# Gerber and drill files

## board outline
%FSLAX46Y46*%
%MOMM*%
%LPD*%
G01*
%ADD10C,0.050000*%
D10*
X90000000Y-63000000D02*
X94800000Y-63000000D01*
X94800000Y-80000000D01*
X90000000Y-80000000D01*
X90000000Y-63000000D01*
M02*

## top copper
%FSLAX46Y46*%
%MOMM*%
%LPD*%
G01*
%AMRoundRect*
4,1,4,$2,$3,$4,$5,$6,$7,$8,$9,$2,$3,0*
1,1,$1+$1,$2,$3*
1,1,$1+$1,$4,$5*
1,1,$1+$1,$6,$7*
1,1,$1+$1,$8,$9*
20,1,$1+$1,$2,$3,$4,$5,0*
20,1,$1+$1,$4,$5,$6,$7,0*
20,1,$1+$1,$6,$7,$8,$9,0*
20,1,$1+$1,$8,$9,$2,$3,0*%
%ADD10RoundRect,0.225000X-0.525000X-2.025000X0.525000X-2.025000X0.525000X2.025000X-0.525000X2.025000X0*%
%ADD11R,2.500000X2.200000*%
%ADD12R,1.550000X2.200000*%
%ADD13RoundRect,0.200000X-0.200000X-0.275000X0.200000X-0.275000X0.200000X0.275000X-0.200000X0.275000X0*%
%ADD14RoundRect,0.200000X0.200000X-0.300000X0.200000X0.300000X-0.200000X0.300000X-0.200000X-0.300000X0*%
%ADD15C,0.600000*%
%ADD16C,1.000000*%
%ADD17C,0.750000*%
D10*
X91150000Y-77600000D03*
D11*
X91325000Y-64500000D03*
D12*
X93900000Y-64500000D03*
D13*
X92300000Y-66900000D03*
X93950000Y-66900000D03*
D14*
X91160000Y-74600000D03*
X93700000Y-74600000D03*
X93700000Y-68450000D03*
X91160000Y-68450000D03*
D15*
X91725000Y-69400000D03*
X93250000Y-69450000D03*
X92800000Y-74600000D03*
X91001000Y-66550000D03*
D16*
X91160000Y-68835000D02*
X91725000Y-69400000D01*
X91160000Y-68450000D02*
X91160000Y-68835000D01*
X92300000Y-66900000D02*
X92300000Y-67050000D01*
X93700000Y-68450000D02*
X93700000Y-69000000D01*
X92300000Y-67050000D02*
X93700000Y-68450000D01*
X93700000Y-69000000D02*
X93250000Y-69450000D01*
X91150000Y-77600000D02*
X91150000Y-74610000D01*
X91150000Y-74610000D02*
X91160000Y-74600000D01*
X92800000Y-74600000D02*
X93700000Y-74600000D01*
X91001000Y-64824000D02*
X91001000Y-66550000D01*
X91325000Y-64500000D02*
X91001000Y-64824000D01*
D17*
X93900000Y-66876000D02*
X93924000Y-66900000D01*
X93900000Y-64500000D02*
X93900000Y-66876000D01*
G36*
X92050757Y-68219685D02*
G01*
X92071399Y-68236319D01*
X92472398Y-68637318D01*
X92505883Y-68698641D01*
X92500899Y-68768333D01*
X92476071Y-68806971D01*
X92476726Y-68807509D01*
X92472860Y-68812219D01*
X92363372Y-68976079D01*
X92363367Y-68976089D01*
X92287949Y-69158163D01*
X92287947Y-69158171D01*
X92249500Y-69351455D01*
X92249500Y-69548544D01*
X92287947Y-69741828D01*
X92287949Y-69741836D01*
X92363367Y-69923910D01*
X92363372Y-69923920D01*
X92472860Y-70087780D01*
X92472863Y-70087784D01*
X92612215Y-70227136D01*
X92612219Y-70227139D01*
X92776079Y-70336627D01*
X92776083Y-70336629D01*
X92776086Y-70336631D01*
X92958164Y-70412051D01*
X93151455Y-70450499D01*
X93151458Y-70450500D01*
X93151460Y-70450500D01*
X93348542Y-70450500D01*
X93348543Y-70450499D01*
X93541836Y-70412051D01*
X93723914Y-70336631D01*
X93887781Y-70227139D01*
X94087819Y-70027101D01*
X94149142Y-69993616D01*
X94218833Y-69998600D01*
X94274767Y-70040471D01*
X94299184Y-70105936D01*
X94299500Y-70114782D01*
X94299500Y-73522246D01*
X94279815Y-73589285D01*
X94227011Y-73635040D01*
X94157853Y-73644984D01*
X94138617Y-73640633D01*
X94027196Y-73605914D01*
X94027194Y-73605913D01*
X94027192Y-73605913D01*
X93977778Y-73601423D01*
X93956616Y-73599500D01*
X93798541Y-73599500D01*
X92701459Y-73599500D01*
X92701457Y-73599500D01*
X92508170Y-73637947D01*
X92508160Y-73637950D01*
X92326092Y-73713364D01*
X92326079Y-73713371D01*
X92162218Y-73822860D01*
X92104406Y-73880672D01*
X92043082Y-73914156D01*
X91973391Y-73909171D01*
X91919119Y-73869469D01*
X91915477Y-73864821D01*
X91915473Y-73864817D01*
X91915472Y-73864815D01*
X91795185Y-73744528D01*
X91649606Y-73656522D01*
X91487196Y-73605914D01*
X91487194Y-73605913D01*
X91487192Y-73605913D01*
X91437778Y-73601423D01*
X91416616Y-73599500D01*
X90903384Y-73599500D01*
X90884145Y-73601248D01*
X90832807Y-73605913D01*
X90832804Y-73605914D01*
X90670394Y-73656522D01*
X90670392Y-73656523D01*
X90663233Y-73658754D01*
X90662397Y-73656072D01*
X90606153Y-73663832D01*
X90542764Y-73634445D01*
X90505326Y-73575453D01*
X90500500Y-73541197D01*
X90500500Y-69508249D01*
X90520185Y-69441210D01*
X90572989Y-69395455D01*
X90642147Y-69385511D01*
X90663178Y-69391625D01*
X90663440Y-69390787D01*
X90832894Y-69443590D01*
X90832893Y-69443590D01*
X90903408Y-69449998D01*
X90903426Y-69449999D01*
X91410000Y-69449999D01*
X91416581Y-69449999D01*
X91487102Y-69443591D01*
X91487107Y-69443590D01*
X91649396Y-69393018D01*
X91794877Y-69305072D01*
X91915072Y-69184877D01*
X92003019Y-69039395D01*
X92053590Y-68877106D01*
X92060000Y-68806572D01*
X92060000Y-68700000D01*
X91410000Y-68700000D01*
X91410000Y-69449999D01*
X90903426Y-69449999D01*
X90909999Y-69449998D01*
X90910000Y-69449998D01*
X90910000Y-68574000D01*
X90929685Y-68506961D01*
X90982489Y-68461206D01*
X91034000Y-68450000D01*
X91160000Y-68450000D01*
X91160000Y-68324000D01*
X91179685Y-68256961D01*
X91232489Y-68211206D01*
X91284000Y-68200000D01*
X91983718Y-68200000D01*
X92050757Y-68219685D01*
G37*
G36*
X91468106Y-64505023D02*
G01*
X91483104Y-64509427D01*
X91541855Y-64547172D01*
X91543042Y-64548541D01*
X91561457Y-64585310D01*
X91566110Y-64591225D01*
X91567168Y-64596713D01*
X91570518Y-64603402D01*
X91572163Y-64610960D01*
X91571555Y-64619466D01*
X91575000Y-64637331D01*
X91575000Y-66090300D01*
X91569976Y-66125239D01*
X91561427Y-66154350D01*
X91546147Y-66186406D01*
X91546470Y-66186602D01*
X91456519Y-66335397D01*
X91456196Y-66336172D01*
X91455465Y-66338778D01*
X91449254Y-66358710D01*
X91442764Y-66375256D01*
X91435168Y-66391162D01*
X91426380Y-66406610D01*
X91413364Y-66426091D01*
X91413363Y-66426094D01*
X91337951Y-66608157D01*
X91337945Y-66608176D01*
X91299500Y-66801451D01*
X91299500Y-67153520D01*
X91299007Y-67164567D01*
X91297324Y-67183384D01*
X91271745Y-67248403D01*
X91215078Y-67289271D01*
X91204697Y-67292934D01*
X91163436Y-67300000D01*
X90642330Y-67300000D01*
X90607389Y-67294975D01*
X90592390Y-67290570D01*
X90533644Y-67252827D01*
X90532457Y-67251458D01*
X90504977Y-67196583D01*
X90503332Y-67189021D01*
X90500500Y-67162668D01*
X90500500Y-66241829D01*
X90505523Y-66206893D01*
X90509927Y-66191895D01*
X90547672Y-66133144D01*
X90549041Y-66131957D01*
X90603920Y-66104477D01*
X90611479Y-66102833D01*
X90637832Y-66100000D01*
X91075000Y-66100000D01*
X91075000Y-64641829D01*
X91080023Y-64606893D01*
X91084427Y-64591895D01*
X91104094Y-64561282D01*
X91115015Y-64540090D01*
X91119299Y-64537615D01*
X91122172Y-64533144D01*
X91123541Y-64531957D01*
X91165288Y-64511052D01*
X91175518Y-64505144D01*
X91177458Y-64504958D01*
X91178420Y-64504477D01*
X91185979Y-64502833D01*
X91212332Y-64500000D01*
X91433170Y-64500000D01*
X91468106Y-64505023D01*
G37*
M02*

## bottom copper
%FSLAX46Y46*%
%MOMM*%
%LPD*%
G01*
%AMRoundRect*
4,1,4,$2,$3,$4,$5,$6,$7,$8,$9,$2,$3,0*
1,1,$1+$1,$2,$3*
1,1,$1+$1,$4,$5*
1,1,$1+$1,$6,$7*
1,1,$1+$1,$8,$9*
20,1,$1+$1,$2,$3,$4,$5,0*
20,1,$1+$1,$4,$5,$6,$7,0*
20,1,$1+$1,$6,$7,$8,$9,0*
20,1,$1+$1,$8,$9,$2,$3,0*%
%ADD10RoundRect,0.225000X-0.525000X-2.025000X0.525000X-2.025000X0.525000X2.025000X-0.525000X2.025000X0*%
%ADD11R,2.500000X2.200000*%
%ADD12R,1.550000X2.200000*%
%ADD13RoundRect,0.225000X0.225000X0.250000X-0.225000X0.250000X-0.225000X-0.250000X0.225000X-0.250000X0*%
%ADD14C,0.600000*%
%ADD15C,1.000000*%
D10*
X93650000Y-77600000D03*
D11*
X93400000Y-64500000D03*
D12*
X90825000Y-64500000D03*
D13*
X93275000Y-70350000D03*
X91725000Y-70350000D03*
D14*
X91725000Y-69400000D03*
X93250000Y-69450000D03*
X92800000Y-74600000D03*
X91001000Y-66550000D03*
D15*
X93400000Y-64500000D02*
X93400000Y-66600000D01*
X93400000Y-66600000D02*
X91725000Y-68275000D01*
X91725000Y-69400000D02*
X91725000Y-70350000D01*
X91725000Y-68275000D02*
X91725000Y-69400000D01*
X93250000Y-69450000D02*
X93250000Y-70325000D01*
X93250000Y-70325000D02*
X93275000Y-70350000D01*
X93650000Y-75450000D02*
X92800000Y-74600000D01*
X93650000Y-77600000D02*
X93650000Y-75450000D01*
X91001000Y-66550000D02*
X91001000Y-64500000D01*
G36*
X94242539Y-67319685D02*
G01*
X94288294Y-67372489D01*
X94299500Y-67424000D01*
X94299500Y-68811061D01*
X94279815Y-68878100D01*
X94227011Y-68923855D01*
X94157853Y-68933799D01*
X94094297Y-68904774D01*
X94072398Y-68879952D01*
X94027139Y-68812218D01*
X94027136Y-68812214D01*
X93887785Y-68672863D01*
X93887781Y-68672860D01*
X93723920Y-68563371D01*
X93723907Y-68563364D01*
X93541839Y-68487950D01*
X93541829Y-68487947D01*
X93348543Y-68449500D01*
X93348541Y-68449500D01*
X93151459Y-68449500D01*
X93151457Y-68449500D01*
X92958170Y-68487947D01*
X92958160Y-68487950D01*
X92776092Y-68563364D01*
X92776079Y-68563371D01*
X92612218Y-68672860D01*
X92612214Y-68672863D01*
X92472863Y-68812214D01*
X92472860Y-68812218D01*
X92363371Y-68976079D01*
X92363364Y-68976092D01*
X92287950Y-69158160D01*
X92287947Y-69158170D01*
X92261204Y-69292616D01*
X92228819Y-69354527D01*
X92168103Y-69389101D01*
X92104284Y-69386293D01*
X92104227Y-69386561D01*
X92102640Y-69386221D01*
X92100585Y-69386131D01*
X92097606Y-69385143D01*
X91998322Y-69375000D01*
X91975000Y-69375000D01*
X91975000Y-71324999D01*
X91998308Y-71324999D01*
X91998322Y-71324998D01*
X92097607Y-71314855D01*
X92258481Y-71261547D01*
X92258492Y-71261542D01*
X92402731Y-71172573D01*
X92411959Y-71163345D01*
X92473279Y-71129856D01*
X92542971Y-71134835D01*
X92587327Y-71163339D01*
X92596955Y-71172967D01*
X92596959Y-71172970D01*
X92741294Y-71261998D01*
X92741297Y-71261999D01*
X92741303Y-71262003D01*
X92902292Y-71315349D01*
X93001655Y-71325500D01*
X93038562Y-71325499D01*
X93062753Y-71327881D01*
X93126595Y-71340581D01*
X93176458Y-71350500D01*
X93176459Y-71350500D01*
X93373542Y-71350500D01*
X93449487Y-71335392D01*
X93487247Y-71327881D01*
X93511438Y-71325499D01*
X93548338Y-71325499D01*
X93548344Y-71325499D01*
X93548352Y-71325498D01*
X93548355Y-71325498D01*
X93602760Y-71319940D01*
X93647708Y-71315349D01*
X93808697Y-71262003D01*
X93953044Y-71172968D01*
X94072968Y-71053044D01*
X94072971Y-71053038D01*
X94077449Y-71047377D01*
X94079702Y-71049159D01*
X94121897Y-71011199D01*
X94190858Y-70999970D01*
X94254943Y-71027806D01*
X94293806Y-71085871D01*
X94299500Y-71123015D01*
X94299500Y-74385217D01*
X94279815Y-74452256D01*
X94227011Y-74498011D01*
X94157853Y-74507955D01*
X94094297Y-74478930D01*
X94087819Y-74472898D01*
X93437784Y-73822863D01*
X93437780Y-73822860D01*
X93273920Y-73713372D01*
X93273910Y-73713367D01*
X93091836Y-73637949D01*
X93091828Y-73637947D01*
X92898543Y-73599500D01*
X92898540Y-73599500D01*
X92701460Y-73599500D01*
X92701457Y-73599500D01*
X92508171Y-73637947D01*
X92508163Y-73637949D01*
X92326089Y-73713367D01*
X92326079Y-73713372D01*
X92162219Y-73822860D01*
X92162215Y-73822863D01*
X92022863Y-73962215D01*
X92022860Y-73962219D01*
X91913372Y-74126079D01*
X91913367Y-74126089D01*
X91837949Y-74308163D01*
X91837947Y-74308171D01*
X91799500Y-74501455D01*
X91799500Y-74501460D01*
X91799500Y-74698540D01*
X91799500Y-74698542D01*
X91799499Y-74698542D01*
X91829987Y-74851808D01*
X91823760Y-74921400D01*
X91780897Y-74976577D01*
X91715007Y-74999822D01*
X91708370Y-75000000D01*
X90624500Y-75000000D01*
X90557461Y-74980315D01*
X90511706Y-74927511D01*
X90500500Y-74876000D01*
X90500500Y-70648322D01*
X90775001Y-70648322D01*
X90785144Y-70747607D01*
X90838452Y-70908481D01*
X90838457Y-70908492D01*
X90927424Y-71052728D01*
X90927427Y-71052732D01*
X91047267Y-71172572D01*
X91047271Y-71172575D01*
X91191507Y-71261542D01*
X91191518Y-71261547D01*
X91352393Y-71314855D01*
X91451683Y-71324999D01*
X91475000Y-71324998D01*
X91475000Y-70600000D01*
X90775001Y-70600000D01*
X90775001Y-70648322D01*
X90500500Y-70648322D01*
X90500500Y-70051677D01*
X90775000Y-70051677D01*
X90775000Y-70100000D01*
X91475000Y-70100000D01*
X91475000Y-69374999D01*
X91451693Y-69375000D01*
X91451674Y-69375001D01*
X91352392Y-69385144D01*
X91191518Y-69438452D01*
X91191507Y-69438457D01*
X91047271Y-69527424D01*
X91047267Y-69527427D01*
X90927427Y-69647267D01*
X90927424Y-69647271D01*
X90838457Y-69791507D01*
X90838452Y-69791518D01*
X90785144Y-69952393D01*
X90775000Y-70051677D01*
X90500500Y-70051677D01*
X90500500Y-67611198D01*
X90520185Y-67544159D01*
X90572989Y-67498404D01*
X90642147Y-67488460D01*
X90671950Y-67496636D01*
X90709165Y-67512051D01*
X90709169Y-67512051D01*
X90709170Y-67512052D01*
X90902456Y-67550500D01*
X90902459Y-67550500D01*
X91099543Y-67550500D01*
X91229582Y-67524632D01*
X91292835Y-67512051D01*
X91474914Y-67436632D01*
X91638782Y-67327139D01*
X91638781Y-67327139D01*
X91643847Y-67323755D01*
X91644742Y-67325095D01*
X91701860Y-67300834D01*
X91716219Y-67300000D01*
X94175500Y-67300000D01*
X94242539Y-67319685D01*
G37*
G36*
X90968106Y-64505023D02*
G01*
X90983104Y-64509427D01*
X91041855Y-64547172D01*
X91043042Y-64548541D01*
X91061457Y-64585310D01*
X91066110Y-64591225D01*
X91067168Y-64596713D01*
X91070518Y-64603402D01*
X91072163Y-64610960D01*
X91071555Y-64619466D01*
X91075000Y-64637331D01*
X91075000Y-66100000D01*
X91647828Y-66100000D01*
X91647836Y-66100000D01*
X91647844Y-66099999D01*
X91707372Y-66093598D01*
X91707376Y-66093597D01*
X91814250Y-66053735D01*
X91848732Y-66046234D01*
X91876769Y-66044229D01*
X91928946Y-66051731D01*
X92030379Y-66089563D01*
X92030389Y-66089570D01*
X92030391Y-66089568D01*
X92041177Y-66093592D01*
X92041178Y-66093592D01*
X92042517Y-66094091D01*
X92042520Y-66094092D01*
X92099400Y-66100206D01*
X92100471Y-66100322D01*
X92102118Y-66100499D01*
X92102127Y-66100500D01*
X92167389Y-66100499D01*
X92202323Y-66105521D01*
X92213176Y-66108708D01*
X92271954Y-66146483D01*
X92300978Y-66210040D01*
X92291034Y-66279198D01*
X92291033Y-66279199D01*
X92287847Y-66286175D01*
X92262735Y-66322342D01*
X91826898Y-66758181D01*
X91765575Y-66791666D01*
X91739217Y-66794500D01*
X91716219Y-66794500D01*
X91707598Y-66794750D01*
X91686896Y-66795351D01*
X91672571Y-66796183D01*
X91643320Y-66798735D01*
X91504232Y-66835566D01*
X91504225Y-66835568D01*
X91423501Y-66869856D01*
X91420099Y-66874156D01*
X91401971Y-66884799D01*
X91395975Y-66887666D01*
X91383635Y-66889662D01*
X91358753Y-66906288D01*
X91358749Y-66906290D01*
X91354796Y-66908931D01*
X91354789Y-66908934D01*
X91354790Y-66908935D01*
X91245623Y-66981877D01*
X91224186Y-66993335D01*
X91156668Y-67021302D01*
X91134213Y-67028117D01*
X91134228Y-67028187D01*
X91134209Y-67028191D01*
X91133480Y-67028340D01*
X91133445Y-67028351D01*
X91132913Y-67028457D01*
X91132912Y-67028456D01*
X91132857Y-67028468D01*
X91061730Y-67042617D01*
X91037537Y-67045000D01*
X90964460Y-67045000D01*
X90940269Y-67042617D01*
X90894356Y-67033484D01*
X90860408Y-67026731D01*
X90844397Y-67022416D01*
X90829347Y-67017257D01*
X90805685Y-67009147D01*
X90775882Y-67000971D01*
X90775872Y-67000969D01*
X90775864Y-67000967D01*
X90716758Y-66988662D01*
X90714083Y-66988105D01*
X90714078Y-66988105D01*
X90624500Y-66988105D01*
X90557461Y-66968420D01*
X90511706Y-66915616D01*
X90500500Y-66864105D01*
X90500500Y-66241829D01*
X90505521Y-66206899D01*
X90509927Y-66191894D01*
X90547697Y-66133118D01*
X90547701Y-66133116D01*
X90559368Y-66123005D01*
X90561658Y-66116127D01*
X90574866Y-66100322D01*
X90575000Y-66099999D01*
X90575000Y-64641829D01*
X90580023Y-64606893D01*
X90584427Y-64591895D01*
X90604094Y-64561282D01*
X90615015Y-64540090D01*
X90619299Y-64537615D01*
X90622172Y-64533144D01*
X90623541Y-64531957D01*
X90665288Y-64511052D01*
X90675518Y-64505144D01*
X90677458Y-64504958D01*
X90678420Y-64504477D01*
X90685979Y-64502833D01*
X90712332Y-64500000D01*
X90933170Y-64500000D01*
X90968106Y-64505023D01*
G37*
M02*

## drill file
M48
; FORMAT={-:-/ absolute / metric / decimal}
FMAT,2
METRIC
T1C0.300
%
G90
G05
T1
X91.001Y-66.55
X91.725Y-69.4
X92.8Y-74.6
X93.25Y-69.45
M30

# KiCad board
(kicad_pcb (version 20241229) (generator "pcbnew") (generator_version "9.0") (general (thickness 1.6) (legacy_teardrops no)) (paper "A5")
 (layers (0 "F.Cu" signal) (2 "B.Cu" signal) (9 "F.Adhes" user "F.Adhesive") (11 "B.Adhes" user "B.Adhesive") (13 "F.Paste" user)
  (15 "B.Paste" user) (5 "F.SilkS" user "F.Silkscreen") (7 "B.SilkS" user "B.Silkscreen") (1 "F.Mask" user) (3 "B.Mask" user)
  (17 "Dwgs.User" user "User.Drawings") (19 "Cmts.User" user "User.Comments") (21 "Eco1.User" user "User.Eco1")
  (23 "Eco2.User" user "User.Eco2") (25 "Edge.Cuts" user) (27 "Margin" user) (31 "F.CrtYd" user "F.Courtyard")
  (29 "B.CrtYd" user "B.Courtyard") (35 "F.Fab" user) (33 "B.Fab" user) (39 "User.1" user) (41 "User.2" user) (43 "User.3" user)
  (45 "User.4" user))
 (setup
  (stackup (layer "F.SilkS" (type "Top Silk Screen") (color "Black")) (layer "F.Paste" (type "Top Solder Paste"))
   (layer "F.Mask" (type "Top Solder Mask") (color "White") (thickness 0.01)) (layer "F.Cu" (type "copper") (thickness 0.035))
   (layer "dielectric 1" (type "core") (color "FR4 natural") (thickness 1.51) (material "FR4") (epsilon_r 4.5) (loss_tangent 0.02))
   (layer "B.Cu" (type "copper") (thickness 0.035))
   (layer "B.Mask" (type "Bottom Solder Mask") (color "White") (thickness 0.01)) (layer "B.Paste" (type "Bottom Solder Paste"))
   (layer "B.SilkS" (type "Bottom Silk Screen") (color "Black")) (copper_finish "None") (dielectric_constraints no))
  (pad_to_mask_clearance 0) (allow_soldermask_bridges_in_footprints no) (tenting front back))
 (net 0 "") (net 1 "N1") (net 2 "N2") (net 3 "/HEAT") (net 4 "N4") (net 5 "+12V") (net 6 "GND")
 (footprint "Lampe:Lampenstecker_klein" (layer "F.Cu") (at 92.4 74.1)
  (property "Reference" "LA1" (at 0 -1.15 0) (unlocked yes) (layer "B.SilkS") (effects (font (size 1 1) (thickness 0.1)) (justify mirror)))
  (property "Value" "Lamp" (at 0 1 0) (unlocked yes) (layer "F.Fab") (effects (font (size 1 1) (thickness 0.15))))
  (pad "1" smd roundrect (at -1.25 3.5) (size 1.5 4.5) (layers "F.Cu" "F.Mask") (roundrect_rratio 0.15) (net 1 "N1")
   (thermal_bridge_angle 45))
  (pad "2" smd roundrect (at 1.25 3.5) (size 1.5 4.5) (layers "B.Cu" "B.Mask") (roundrect_rratio 0.15) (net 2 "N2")
   (thermal_bridge_angle 45)))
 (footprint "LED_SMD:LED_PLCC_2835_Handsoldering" (layer "F.Cu") (at 92.375 64.5)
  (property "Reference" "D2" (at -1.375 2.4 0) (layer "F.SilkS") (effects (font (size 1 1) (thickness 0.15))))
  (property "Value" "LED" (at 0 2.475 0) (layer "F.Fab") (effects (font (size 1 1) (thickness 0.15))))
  (pad "1" smd rect (at -1.05 0) (size 2.5 2.2) (layers "F.Cu" "F.Mask" "F.Paste") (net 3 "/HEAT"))
  (pad "2" smd rect (at 1.525 0) (size 1.55 2.2) (layers "F.Cu" "F.Mask" "F.Paste") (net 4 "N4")))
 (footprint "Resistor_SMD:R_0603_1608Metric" (layer "F.Cu") (at 93.125 66.9)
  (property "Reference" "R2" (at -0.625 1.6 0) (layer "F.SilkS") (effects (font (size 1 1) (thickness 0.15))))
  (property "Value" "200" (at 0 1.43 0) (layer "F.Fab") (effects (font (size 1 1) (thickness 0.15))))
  (pad "1" smd roundrect (at -0.825 0) (size 0.8 0.95) (layers "F.Cu" "F.Mask" "F.Paste") (roundrect_rratio 0.25) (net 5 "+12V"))
  (pad "2" smd roundrect (at 0.825 0) (size 0.8 0.95) (layers "F.Cu" "F.Mask" "F.Paste") (roundrect_rratio 0.25) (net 4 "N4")))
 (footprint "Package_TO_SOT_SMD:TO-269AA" (layer "F.Cu") (at 92.43 71.525 90)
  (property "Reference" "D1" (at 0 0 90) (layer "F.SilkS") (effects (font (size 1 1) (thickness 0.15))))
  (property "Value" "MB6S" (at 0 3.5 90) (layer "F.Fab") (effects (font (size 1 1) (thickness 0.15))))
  (pad "1" smd roundrect (at -3.075 -1.27 90) (size 1 0.8) (layers "F.Cu" "F.Mask" "F.Paste") (roundrect_rratio 0.25) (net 1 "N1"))
  (pad "2" smd roundrect (at -3.075 1.27 90) (size 1 0.8) (layers "F.Cu" "F.Mask" "F.Paste") (roundrect_rratio 0.25) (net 2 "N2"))
  (pad "3" smd roundrect (at 3.075 1.27 90) (size 1 0.8) (layers "F.Cu" "F.Mask" "F.Paste") (roundrect_rratio 0.25) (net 5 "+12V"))
  (pad "4" smd roundrect (at 3.075 -1.27 90) (size 1 0.8) (layers "F.Cu" "F.Mask" "F.Paste") (roundrect_rratio 0.25) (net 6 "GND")))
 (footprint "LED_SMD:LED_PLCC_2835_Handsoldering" (layer "B.Cu") (at 92.35 64.5 180)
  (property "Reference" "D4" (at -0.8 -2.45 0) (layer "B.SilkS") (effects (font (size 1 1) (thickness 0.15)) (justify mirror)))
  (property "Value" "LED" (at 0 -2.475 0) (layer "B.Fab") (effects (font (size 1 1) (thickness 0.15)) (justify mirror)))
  (pad "1" smd rect (at -1.05 0 180) (size 2.5 2.2) (layers "B.Cu" "B.Mask" "B.Paste") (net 6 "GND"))
  (pad "2" smd rect (at 1.525 0 180) (size 1.55 2.2) (layers "B.Cu" "B.Mask" "B.Paste") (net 3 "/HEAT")))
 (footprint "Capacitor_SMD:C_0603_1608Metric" (layer "B.Cu") (at 92.5 70.35 180)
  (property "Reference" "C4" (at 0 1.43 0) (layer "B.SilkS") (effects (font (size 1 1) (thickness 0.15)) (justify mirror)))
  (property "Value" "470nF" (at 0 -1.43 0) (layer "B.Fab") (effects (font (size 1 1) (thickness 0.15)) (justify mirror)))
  (pad "1" smd roundrect (at -0.775 0 180) (size 0.9 0.95) (layers "B.Cu" "B.Mask" "B.Paste") (roundrect_rratio 0.25) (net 5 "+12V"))
  (pad "2" smd roundrect (at 0.775 0 180) (size 0.9 0.95) (layers "B.Cu" "B.Mask" "B.Paste") (roundrect_rratio 0.25) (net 6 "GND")))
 (gr_rect (start 90 63) (end 94.8 80) (stroke (width 0.05) (type default)) (fill no) (layer "Edge.Cuts"))
 (segment (start 91.16 68.835) (end 91.725 69.4) (width 1) (layer "F.Cu") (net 6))
 (segment (start 91.16 68.45) (end 91.16 68.835) (width 1) (layer "F.Cu") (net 6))
 (via (at 91.725 69.4) (size 0.6) (drill 0.3) (layers "F.Cu" "B.Cu") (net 6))
 (segment (start 93.4 64.5) (end 93.4 66.6) (width 1) (layer "B.Cu") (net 6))
 (segment (start 93.4 66.6) (end 91.725 68.275) (width 1) (layer "B.Cu") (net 6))
 (segment (start 91.725 69.4) (end 91.725 70.35) (width 1) (layer "B.Cu") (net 6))
 (segment (start 91.725 68.275) (end 91.725 69.4) (width 1) (layer "B.Cu") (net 6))
 (segment (start 92.3 66.9) (end 92.3 67.05) (width 1) (layer "F.Cu") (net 5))
 (segment (start 93.7 68.45) (end 93.7 69) (width 1) (layer "F.Cu") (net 5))
 (segment (start 92.3 67.05) (end 93.7 68.45) (width 1) (layer "F.Cu") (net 5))
 (segment (start 93.7 69) (end 93.25 69.45) (width 1) (layer "F.Cu") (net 5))
 (via (at 93.25 69.45) (size 0.6) (drill 0.3) (layers "F.Cu" "B.Cu") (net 5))
 (segment (start 93.25 69.45) (end 93.25 70.325) (width 1) (layer "B.Cu") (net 5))
 (segment (start 93.25 70.325) (end 93.275 70.35) (width 1) (layer "B.Cu") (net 5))
 (segment (start 91.15 77.6) (end 91.15 74.61) (width 1) (layer "F.Cu") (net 1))
 (segment (start 91.15 74.61) (end 91.16 74.6) (width 1) (layer "F.Cu") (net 1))
 (segment (start 92.8 74.6) (end 93.7 74.6) (width 1) (layer "F.Cu") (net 2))
 (via (at 92.8 74.6) (size 0.6) (drill 0.3) (layers "F.Cu" "B.Cu") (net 2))
 (segment (start 93.65 75.45) (end 92.8 74.6) (width 1) (layer "B.Cu") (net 2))
 (segment (start 93.65 77.6) (end 93.65 75.45) (width 1) (layer "B.Cu") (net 2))
 (segment (start 91.001 64.824) (end 91.001 66.55) (width 1) (layer "F.Cu") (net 3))
 (segment (start 91.325 64.5) (end 91.001 64.824) (width 1) (layer "F.Cu") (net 3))
 (via (at 91.001 66.55) (size 0.6) (drill 0.3) (layers "F.Cu" "B.Cu") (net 3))
 (segment (start 91.001 66.55) (end 91.001 64.5) (width 1) (layer "B.Cu") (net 3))
 (segment (start 93.9 66.876) (end 93.924 66.9) (width 0.75) (layer "F.Cu") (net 4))
 (segment (start 93.9 64.5) (end 93.9 66.876) (width 0.75) (layer "F.Cu") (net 4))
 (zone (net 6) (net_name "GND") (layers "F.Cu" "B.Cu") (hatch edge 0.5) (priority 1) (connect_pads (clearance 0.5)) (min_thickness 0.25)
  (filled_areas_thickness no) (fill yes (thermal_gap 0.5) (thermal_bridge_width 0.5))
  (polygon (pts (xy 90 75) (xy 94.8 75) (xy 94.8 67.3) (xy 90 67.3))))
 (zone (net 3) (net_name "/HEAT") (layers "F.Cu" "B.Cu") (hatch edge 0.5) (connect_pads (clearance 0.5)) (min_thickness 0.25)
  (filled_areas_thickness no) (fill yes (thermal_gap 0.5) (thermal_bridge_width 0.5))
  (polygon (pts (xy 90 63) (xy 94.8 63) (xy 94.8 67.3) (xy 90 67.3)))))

